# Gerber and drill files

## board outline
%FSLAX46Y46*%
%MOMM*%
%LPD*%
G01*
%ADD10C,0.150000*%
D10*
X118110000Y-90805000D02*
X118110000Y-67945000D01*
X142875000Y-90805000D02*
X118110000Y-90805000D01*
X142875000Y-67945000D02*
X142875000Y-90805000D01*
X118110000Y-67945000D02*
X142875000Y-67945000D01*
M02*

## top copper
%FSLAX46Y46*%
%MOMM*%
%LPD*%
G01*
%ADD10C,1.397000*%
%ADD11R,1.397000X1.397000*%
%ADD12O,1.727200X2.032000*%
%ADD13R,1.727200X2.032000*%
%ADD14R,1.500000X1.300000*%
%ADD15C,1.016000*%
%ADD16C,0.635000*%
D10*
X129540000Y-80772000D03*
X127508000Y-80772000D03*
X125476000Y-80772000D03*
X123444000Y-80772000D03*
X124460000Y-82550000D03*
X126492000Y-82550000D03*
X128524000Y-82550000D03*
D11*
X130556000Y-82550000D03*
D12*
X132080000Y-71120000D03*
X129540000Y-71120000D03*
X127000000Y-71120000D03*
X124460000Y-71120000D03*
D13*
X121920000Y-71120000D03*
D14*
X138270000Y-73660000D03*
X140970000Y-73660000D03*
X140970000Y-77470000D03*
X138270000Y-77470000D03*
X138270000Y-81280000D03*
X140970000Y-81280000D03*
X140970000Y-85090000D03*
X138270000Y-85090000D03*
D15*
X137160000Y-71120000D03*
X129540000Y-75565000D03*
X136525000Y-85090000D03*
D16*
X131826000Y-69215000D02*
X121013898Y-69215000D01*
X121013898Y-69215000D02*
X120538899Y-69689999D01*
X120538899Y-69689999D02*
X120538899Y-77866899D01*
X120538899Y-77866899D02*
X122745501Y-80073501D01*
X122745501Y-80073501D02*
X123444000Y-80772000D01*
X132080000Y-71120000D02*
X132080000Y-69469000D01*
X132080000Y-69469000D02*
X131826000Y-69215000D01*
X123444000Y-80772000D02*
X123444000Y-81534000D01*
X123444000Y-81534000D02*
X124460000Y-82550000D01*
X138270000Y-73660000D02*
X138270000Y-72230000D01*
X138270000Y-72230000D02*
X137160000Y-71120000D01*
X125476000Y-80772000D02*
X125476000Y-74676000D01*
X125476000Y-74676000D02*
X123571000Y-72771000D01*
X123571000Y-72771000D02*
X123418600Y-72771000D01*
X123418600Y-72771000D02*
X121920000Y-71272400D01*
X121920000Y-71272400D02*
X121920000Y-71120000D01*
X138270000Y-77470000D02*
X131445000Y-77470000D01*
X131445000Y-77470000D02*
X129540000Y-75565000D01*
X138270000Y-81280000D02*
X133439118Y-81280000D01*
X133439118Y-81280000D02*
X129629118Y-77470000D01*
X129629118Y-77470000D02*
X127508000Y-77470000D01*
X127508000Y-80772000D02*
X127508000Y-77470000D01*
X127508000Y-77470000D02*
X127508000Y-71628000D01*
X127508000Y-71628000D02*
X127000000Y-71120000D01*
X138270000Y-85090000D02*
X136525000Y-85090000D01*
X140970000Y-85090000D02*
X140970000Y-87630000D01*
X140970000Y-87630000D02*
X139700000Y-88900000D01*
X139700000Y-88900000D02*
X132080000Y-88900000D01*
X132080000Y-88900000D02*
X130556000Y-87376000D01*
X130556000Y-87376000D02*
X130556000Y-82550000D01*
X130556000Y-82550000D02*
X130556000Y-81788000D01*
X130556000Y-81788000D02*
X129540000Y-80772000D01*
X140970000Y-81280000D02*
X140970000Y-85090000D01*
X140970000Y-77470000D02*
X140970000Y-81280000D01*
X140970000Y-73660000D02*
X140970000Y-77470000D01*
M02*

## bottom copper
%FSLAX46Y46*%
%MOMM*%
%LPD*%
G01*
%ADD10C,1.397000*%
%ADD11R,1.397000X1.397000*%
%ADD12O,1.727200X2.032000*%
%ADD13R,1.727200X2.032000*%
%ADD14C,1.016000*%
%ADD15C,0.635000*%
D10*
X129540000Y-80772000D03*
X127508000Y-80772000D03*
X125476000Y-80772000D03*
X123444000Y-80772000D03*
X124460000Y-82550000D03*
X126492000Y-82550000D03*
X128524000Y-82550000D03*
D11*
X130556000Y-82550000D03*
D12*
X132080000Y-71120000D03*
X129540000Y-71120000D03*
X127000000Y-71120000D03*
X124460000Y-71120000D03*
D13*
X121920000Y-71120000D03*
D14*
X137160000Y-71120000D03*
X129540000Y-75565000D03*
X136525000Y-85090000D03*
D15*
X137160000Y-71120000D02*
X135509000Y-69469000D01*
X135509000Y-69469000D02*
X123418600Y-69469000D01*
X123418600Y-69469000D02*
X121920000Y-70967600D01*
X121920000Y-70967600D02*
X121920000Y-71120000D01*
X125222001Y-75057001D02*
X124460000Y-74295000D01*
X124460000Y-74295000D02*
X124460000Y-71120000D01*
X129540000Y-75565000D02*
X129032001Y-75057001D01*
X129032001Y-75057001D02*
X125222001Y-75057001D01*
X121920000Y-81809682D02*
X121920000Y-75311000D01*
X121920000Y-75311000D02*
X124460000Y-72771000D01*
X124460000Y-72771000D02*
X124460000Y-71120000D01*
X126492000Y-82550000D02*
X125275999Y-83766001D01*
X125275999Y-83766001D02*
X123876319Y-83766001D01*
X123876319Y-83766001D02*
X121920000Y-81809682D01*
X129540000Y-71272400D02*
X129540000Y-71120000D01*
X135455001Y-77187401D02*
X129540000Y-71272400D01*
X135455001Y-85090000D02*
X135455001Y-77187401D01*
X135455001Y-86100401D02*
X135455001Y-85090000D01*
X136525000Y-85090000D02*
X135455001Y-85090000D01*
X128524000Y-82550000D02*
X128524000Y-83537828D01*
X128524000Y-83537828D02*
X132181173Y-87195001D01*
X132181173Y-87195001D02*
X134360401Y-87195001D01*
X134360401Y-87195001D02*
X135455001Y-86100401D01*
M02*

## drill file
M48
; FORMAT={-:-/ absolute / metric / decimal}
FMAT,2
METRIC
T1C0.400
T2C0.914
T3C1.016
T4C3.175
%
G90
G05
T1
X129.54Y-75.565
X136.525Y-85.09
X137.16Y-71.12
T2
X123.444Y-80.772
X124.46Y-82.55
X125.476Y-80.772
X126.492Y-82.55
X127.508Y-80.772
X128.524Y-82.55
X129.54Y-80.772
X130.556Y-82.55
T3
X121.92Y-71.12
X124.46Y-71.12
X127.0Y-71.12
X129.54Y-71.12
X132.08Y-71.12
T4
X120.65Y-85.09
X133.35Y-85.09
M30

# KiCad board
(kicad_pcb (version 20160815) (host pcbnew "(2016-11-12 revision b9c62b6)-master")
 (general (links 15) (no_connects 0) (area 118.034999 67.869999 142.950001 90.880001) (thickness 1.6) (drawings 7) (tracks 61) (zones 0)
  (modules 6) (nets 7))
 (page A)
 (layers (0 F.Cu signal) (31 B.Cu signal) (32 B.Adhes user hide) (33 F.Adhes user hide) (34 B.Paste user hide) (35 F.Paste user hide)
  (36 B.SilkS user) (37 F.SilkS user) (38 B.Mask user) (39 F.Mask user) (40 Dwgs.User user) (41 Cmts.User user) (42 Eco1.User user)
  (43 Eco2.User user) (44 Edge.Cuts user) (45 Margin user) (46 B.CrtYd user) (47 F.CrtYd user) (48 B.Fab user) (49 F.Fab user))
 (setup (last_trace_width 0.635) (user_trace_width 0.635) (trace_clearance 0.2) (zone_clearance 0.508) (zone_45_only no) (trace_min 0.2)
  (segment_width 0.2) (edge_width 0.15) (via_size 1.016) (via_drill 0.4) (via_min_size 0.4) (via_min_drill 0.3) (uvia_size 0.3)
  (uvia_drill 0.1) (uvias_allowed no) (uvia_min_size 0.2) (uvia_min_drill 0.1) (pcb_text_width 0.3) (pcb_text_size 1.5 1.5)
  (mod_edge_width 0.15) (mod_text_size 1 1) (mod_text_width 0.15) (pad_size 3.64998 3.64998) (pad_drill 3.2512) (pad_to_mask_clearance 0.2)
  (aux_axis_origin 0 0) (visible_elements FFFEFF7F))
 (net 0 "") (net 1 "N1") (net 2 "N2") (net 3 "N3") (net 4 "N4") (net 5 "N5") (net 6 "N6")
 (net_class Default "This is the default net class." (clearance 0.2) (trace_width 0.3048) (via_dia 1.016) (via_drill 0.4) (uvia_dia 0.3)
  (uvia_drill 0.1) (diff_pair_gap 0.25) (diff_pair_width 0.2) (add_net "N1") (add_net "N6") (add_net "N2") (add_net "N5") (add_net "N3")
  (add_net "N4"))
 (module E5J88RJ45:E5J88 (layer F.Cu) (at 127 85.09)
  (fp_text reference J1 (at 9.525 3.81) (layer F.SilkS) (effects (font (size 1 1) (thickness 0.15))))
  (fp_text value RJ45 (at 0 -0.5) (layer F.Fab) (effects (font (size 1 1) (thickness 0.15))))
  (pad 2 thru_hole circle (at 2.54 -4.318) (size 1.397 1.397) (drill 0.9144) (layers *.Cu *.Mask) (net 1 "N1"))
  (pad 4 thru_hole circle (at 0.508 -4.318) (size 1.397 1.397) (drill 0.9144) (layers *.Cu *.Mask) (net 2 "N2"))
  (pad 6 thru_hole circle (at -1.524 -4.318) (size 1.397 1.397) (drill 0.9144) (layers *.Cu *.Mask) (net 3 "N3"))
  (pad 8 thru_hole circle (at -3.556 -4.318) (size 1.397 1.397) (drill 0.9144) (layers *.Cu *.Mask) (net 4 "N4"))
  (pad 7 thru_hole circle (at -2.54 -2.54) (size 1.397 1.397) (drill 0.9144) (layers *.Cu *.Mask) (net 4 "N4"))
  (pad 5 thru_hole circle (at -0.508 -2.54) (size 1.397 1.397) (drill 0.9144) (layers *.Cu *.Mask) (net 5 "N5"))
  (pad 3 thru_hole circle (at 1.524 -2.54) (size 1.397 1.397) (drill 0.9144) (layers *.Cu *.Mask) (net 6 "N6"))
  (pad 1 thru_hole rect (at 3.556 -2.54) (size 1.397 1.397) (drill 0.9144) (layers *.Cu *.Mask) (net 1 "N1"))
  (pad "" np_thru_hole circle (at 6.35 0) (size 3.175 3.175) (drill 3.175) (layers *.Cu *.Mask))
  (pad "" np_thru_hole circle (at -6.35 0) (size 3.175 3.175) (drill 3.175) (layers *.Cu *.Mask)))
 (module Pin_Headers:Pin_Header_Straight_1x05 (layer F.Cu) (at 121.92 71.12 90)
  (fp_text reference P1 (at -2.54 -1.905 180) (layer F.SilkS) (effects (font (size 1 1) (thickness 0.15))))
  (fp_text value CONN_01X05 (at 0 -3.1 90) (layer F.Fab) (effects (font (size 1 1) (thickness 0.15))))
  (pad 5 thru_hole oval (at 0 10.16 90) (size 2.032 1.7272) (drill 1.016) (layers *.Cu *.Mask) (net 4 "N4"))
  (pad 4 thru_hole oval (at 0 7.62 90) (size 2.032 1.7272) (drill 1.016) (layers *.Cu *.Mask) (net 6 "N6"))
  (pad 3 thru_hole oval (at 0 5.08 90) (size 2.032 1.7272) (drill 1.016) (layers *.Cu *.Mask) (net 2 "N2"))
  (pad 2 thru_hole oval (at 0 2.54 90) (size 2.032 1.7272) (drill 1.016) (layers *.Cu *.Mask) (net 5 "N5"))
  (pad 1 thru_hole rect (at 0 0 90) (size 2.032 1.7272) (drill 1.016) (layers *.Cu *.Mask) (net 3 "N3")))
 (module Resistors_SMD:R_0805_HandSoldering (layer F.Cu) (at 139.62 73.66 180)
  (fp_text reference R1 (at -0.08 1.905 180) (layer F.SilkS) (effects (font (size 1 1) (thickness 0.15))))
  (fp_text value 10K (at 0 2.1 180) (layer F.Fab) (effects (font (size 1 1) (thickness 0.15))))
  (pad 2 smd rect (at 1.35 0 180) (size 1.5 1.3) (layers F.Cu F.Paste F.Mask) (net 3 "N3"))
  (pad 1 smd rect (at -1.35 0 180) (size 1.5 1.3) (layers F.Cu F.Paste F.Mask) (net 1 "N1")))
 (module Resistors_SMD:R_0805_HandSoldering (layer F.Cu) (at 139.62 77.47 180)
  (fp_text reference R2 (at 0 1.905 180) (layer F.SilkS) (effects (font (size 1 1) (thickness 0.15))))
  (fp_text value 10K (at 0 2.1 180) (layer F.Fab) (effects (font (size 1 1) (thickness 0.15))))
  (pad 1 smd rect (at -1.35 0 180) (size 1.5 1.3) (layers F.Cu F.Paste F.Mask) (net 1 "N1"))
  (pad 2 smd rect (at 1.35 0 180) (size 1.5 1.3) (layers F.Cu F.Paste F.Mask) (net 5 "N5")))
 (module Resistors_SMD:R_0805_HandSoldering (layer F.Cu) (at 139.62 81.28 180)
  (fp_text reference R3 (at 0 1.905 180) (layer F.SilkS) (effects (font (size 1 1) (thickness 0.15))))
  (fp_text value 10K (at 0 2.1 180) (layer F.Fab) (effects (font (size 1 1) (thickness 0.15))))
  (pad 2 smd rect (at 1.35 0 180) (size 1.5 1.3) (layers F.Cu F.Paste F.Mask) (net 2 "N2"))
  (pad 1 smd rect (at -1.35 0 180) (size 1.5 1.3) (layers F.Cu F.Paste F.Mask) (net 1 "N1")))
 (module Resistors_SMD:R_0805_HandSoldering (layer F.Cu) (at 139.62 85.09 180)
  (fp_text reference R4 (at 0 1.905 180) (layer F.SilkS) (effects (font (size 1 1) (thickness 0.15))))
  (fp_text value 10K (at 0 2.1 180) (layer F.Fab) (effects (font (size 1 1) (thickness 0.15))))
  (pad 1 smd rect (at -1.35 0 180) (size 1.5 1.3) (layers F.Cu F.Paste F.Mask) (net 1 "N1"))
  (pad 2 smd rect (at 1.35 0 180) (size 1.5 1.3) (layers F.Cu F.Paste F.Mask) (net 6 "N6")))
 (gr_line (start 118.11 90.805) (end 118.11 67.945) (layer Edge.Cuts) (width 0.15))
 (gr_line (start 142.875 90.805) (end 118.11 90.805) (layer Edge.Cuts) (width 0.15))
 (gr_line (start 142.875 67.945) (end 142.875 90.805) (layer Edge.Cuts) (width 0.15))
 (gr_line (start 118.11 67.945) (end 142.875 67.945) (layer Edge.Cuts) (width 0.15))
 (segment (start 131.826 69.215) (end 121.013898 69.215) (width 0.635) (layer F.Cu) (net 4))
 (segment (start 121.013898 69.215) (end 120.538899 69.689999) (width 0.635) (layer F.Cu) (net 4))
 (segment (start 120.538899 69.689999) (end 120.538899 77.866899) (width 0.635) (layer F.Cu) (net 4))
 (segment (start 120.538899 77.866899) (end 122.745501 80.073501) (width 0.635) (layer F.Cu) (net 4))
 (segment (start 122.745501 80.073501) (end 123.444 80.772) (width 0.635) (layer F.Cu) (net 4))
 (segment (start 132.08 71.12) (end 132.08 69.469) (width 0.635) (layer F.Cu) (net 4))
 (segment (start 132.08 69.469) (end 131.826 69.215) (width 0.635) (layer F.Cu) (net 4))
 (segment (start 123.444 80.772) (end 123.444 81.534) (width 0.635) (layer F.Cu) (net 4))
 (segment (start 123.444 81.534) (end 124.46 82.55) (width 0.635) (layer F.Cu) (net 4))
 (segment (start 137.16 71.12) (end 135.509 69.469) (width 0.635) (layer B.Cu) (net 3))
 (segment (start 135.509 69.469) (end 123.4186 69.469) (width 0.635) (layer B.Cu) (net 3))
 (segment (start 123.4186 69.469) (end 121.92 70.9676) (width 0.635) (layer B.Cu) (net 3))
 (segment (start 121.92 70.9676) (end 121.92 71.12) (width 0.635) (layer B.Cu) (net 3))
 (segment (start 138.27 73.66) (end 138.27 72.23) (width 0.635) (layer F.Cu) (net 3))
 (segment (start 138.27 72.23) (end 137.16 71.12) (width 0.635) (layer F.Cu) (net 3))
 (via (at 137.16 71.12) (size 1.016) (drill 0.4) (layers F.Cu B.Cu) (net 3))
 (segment (start 125.476 80.772) (end 125.476 74.676) (width 0.635) (layer F.Cu) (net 3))
 (segment (start 125.476 74.676) (end 123.571 72.771) (width 0.635) (layer F.Cu) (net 3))
 (segment (start 123.571 72.771) (end 123.4186 72.771) (width 0.635) (layer F.Cu) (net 3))
 (segment (start 123.4186 72.771) (end 121.92 71.2724) (width 0.635) (layer F.Cu) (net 3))
 (segment (start 121.92 71.2724) (end 121.92 71.12) (width 0.635) (layer F.Cu) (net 3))
 (segment (start 125.222001 75.057001) (end 124.46 74.295) (width 0.635) (layer B.Cu) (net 5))
 (segment (start 124.46 74.295) (end 124.46 71.12) (width 0.635) (layer B.Cu) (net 5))
 (segment (start 129.54 75.565) (end 129.032001 75.057001) (width 0.635) (layer B.Cu) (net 5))
 (segment (start 129.032001 75.057001) (end 125.222001 75.057001) (width 0.635) (layer B.Cu) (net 5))
 (segment (start 138.27 77.47) (end 131.445 77.47) (width 0.635) (layer F.Cu) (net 5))
 (segment (start 131.445 77.47) (end 129.54 75.565) (width 0.635) (layer F.Cu) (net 5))
 (via (at 129.54 75.565) (size 1.016) (drill 0.4) (layers F.Cu B.Cu) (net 5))
 (segment (start 121.92 81.809682) (end 121.92 75.311) (width 0.635) (layer B.Cu) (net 5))
 (segment (start 121.92 75.311) (end 124.46 72.771) (width 0.635) (layer B.Cu) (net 5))
 (segment (start 124.46 72.771) (end 124.46 71.12) (width 0.635) (layer B.Cu) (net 5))
 (segment (start 126.492 82.55) (end 125.275999 83.766001) (width 0.635) (layer B.Cu) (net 5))
 (segment (start 125.275999 83.766001) (end 123.876319 83.766001) (width 0.635) (layer B.Cu) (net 5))
 (segment (start 123.876319 83.766001) (end 121.92 81.809682) (width 0.635) (layer B.Cu) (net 5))
 (segment (start 138.27 81.28) (end 133.439118 81.28) (width 0.635) (layer F.Cu) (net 2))
 (segment (start 133.439118 81.28) (end 129.629118 77.47) (width 0.635) (layer F.Cu) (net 2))
 (segment (start 129.629118 77.47) (end 127.508 77.47) (width 0.635) (layer F.Cu) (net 2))
 (segment (start 127.508 80.772) (end 127.508 77.47) (width 0.635) (layer F.Cu) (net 2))
 (segment (start 127.508 77.47) (end 127.508 71.628) (width 0.635) (layer F.Cu) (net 2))
 (segment (start 127.508 71.628) (end 127 71.12) (width 0.635) (layer F.Cu) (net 2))
 (segment (start 129.54 71.2724) (end 129.54 71.12) (width 0.635) (layer B.Cu) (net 6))
 (segment (start 135.455001 77.187401) (end 129.54 71.2724) (width 0.635) (layer B.Cu) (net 6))
 (segment (start 135.455001 85.09) (end 135.455001 77.187401) (width 0.635) (layer B.Cu) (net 6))
 (segment (start 135.455001 86.100401) (end 135.455001 85.09) (width 0.635) (layer B.Cu) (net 6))
 (segment (start 136.525 85.09) (end 135.455001 85.09) (width 0.635) (layer B.Cu) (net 6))
 (segment (start 138.27 85.09) (end 136.525 85.09) (width 0.635) (layer F.Cu) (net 6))
 (via (at 136.525 85.09) (size 1.016) (drill 0.4) (layers F.Cu B.Cu) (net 6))
 (segment (start 128.524 82.55) (end 128.524 83.537828) (width 0.635) (layer B.Cu) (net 6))
 (segment (start 128.524 83.537828) (end 132.181173 87.195001) (width 0.635) (layer B.Cu) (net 6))
 (segment (start 132.181173 87.195001) (end 134.360401 87.195001) (width 0.635) (layer B.Cu) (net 6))
 (segment (start 134.360401 87.195001) (end 135.455001 86.100401) (width 0.635) (layer B.Cu) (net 6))
 (segment (start 140.97 85.09) (end 140.97 87.63) (width 0.635) (layer F.Cu) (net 1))
 (segment (start 140.97 87.63) (end 139.7 88.9) (width 0.635) (layer F.Cu) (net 1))
 (segment (start 139.7 88.9) (end 132.08 88.9) (width 0.635) (layer F.Cu) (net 1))
 (segment (start 132.08 88.9) (end 130.556 87.376) (width 0.635) (layer F.Cu) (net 1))
 (segment (start 130.556 87.376) (end 130.556 82.55) (width 0.635) (layer F.Cu) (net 1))
 (segment (start 130.556 82.55) (end 130.556 81.788) (width 0.635) (layer F.Cu) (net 1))
 (segment (start 130.556 81.788) (end 129.54 80.772) (width 0.635) (layer F.Cu) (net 1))
 (segment (start 140.97 81.28) (end 140.97 85.09) (width 0.635) (layer F.Cu) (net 1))
 (segment (start 140.97 77.47) (end 140.97 81.28) (width 0.635) (layer F.Cu) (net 1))
 (segment (start 140.97 73.66) (end 140.97 77.47) (width 0.635) (layer F.Cu) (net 1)))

